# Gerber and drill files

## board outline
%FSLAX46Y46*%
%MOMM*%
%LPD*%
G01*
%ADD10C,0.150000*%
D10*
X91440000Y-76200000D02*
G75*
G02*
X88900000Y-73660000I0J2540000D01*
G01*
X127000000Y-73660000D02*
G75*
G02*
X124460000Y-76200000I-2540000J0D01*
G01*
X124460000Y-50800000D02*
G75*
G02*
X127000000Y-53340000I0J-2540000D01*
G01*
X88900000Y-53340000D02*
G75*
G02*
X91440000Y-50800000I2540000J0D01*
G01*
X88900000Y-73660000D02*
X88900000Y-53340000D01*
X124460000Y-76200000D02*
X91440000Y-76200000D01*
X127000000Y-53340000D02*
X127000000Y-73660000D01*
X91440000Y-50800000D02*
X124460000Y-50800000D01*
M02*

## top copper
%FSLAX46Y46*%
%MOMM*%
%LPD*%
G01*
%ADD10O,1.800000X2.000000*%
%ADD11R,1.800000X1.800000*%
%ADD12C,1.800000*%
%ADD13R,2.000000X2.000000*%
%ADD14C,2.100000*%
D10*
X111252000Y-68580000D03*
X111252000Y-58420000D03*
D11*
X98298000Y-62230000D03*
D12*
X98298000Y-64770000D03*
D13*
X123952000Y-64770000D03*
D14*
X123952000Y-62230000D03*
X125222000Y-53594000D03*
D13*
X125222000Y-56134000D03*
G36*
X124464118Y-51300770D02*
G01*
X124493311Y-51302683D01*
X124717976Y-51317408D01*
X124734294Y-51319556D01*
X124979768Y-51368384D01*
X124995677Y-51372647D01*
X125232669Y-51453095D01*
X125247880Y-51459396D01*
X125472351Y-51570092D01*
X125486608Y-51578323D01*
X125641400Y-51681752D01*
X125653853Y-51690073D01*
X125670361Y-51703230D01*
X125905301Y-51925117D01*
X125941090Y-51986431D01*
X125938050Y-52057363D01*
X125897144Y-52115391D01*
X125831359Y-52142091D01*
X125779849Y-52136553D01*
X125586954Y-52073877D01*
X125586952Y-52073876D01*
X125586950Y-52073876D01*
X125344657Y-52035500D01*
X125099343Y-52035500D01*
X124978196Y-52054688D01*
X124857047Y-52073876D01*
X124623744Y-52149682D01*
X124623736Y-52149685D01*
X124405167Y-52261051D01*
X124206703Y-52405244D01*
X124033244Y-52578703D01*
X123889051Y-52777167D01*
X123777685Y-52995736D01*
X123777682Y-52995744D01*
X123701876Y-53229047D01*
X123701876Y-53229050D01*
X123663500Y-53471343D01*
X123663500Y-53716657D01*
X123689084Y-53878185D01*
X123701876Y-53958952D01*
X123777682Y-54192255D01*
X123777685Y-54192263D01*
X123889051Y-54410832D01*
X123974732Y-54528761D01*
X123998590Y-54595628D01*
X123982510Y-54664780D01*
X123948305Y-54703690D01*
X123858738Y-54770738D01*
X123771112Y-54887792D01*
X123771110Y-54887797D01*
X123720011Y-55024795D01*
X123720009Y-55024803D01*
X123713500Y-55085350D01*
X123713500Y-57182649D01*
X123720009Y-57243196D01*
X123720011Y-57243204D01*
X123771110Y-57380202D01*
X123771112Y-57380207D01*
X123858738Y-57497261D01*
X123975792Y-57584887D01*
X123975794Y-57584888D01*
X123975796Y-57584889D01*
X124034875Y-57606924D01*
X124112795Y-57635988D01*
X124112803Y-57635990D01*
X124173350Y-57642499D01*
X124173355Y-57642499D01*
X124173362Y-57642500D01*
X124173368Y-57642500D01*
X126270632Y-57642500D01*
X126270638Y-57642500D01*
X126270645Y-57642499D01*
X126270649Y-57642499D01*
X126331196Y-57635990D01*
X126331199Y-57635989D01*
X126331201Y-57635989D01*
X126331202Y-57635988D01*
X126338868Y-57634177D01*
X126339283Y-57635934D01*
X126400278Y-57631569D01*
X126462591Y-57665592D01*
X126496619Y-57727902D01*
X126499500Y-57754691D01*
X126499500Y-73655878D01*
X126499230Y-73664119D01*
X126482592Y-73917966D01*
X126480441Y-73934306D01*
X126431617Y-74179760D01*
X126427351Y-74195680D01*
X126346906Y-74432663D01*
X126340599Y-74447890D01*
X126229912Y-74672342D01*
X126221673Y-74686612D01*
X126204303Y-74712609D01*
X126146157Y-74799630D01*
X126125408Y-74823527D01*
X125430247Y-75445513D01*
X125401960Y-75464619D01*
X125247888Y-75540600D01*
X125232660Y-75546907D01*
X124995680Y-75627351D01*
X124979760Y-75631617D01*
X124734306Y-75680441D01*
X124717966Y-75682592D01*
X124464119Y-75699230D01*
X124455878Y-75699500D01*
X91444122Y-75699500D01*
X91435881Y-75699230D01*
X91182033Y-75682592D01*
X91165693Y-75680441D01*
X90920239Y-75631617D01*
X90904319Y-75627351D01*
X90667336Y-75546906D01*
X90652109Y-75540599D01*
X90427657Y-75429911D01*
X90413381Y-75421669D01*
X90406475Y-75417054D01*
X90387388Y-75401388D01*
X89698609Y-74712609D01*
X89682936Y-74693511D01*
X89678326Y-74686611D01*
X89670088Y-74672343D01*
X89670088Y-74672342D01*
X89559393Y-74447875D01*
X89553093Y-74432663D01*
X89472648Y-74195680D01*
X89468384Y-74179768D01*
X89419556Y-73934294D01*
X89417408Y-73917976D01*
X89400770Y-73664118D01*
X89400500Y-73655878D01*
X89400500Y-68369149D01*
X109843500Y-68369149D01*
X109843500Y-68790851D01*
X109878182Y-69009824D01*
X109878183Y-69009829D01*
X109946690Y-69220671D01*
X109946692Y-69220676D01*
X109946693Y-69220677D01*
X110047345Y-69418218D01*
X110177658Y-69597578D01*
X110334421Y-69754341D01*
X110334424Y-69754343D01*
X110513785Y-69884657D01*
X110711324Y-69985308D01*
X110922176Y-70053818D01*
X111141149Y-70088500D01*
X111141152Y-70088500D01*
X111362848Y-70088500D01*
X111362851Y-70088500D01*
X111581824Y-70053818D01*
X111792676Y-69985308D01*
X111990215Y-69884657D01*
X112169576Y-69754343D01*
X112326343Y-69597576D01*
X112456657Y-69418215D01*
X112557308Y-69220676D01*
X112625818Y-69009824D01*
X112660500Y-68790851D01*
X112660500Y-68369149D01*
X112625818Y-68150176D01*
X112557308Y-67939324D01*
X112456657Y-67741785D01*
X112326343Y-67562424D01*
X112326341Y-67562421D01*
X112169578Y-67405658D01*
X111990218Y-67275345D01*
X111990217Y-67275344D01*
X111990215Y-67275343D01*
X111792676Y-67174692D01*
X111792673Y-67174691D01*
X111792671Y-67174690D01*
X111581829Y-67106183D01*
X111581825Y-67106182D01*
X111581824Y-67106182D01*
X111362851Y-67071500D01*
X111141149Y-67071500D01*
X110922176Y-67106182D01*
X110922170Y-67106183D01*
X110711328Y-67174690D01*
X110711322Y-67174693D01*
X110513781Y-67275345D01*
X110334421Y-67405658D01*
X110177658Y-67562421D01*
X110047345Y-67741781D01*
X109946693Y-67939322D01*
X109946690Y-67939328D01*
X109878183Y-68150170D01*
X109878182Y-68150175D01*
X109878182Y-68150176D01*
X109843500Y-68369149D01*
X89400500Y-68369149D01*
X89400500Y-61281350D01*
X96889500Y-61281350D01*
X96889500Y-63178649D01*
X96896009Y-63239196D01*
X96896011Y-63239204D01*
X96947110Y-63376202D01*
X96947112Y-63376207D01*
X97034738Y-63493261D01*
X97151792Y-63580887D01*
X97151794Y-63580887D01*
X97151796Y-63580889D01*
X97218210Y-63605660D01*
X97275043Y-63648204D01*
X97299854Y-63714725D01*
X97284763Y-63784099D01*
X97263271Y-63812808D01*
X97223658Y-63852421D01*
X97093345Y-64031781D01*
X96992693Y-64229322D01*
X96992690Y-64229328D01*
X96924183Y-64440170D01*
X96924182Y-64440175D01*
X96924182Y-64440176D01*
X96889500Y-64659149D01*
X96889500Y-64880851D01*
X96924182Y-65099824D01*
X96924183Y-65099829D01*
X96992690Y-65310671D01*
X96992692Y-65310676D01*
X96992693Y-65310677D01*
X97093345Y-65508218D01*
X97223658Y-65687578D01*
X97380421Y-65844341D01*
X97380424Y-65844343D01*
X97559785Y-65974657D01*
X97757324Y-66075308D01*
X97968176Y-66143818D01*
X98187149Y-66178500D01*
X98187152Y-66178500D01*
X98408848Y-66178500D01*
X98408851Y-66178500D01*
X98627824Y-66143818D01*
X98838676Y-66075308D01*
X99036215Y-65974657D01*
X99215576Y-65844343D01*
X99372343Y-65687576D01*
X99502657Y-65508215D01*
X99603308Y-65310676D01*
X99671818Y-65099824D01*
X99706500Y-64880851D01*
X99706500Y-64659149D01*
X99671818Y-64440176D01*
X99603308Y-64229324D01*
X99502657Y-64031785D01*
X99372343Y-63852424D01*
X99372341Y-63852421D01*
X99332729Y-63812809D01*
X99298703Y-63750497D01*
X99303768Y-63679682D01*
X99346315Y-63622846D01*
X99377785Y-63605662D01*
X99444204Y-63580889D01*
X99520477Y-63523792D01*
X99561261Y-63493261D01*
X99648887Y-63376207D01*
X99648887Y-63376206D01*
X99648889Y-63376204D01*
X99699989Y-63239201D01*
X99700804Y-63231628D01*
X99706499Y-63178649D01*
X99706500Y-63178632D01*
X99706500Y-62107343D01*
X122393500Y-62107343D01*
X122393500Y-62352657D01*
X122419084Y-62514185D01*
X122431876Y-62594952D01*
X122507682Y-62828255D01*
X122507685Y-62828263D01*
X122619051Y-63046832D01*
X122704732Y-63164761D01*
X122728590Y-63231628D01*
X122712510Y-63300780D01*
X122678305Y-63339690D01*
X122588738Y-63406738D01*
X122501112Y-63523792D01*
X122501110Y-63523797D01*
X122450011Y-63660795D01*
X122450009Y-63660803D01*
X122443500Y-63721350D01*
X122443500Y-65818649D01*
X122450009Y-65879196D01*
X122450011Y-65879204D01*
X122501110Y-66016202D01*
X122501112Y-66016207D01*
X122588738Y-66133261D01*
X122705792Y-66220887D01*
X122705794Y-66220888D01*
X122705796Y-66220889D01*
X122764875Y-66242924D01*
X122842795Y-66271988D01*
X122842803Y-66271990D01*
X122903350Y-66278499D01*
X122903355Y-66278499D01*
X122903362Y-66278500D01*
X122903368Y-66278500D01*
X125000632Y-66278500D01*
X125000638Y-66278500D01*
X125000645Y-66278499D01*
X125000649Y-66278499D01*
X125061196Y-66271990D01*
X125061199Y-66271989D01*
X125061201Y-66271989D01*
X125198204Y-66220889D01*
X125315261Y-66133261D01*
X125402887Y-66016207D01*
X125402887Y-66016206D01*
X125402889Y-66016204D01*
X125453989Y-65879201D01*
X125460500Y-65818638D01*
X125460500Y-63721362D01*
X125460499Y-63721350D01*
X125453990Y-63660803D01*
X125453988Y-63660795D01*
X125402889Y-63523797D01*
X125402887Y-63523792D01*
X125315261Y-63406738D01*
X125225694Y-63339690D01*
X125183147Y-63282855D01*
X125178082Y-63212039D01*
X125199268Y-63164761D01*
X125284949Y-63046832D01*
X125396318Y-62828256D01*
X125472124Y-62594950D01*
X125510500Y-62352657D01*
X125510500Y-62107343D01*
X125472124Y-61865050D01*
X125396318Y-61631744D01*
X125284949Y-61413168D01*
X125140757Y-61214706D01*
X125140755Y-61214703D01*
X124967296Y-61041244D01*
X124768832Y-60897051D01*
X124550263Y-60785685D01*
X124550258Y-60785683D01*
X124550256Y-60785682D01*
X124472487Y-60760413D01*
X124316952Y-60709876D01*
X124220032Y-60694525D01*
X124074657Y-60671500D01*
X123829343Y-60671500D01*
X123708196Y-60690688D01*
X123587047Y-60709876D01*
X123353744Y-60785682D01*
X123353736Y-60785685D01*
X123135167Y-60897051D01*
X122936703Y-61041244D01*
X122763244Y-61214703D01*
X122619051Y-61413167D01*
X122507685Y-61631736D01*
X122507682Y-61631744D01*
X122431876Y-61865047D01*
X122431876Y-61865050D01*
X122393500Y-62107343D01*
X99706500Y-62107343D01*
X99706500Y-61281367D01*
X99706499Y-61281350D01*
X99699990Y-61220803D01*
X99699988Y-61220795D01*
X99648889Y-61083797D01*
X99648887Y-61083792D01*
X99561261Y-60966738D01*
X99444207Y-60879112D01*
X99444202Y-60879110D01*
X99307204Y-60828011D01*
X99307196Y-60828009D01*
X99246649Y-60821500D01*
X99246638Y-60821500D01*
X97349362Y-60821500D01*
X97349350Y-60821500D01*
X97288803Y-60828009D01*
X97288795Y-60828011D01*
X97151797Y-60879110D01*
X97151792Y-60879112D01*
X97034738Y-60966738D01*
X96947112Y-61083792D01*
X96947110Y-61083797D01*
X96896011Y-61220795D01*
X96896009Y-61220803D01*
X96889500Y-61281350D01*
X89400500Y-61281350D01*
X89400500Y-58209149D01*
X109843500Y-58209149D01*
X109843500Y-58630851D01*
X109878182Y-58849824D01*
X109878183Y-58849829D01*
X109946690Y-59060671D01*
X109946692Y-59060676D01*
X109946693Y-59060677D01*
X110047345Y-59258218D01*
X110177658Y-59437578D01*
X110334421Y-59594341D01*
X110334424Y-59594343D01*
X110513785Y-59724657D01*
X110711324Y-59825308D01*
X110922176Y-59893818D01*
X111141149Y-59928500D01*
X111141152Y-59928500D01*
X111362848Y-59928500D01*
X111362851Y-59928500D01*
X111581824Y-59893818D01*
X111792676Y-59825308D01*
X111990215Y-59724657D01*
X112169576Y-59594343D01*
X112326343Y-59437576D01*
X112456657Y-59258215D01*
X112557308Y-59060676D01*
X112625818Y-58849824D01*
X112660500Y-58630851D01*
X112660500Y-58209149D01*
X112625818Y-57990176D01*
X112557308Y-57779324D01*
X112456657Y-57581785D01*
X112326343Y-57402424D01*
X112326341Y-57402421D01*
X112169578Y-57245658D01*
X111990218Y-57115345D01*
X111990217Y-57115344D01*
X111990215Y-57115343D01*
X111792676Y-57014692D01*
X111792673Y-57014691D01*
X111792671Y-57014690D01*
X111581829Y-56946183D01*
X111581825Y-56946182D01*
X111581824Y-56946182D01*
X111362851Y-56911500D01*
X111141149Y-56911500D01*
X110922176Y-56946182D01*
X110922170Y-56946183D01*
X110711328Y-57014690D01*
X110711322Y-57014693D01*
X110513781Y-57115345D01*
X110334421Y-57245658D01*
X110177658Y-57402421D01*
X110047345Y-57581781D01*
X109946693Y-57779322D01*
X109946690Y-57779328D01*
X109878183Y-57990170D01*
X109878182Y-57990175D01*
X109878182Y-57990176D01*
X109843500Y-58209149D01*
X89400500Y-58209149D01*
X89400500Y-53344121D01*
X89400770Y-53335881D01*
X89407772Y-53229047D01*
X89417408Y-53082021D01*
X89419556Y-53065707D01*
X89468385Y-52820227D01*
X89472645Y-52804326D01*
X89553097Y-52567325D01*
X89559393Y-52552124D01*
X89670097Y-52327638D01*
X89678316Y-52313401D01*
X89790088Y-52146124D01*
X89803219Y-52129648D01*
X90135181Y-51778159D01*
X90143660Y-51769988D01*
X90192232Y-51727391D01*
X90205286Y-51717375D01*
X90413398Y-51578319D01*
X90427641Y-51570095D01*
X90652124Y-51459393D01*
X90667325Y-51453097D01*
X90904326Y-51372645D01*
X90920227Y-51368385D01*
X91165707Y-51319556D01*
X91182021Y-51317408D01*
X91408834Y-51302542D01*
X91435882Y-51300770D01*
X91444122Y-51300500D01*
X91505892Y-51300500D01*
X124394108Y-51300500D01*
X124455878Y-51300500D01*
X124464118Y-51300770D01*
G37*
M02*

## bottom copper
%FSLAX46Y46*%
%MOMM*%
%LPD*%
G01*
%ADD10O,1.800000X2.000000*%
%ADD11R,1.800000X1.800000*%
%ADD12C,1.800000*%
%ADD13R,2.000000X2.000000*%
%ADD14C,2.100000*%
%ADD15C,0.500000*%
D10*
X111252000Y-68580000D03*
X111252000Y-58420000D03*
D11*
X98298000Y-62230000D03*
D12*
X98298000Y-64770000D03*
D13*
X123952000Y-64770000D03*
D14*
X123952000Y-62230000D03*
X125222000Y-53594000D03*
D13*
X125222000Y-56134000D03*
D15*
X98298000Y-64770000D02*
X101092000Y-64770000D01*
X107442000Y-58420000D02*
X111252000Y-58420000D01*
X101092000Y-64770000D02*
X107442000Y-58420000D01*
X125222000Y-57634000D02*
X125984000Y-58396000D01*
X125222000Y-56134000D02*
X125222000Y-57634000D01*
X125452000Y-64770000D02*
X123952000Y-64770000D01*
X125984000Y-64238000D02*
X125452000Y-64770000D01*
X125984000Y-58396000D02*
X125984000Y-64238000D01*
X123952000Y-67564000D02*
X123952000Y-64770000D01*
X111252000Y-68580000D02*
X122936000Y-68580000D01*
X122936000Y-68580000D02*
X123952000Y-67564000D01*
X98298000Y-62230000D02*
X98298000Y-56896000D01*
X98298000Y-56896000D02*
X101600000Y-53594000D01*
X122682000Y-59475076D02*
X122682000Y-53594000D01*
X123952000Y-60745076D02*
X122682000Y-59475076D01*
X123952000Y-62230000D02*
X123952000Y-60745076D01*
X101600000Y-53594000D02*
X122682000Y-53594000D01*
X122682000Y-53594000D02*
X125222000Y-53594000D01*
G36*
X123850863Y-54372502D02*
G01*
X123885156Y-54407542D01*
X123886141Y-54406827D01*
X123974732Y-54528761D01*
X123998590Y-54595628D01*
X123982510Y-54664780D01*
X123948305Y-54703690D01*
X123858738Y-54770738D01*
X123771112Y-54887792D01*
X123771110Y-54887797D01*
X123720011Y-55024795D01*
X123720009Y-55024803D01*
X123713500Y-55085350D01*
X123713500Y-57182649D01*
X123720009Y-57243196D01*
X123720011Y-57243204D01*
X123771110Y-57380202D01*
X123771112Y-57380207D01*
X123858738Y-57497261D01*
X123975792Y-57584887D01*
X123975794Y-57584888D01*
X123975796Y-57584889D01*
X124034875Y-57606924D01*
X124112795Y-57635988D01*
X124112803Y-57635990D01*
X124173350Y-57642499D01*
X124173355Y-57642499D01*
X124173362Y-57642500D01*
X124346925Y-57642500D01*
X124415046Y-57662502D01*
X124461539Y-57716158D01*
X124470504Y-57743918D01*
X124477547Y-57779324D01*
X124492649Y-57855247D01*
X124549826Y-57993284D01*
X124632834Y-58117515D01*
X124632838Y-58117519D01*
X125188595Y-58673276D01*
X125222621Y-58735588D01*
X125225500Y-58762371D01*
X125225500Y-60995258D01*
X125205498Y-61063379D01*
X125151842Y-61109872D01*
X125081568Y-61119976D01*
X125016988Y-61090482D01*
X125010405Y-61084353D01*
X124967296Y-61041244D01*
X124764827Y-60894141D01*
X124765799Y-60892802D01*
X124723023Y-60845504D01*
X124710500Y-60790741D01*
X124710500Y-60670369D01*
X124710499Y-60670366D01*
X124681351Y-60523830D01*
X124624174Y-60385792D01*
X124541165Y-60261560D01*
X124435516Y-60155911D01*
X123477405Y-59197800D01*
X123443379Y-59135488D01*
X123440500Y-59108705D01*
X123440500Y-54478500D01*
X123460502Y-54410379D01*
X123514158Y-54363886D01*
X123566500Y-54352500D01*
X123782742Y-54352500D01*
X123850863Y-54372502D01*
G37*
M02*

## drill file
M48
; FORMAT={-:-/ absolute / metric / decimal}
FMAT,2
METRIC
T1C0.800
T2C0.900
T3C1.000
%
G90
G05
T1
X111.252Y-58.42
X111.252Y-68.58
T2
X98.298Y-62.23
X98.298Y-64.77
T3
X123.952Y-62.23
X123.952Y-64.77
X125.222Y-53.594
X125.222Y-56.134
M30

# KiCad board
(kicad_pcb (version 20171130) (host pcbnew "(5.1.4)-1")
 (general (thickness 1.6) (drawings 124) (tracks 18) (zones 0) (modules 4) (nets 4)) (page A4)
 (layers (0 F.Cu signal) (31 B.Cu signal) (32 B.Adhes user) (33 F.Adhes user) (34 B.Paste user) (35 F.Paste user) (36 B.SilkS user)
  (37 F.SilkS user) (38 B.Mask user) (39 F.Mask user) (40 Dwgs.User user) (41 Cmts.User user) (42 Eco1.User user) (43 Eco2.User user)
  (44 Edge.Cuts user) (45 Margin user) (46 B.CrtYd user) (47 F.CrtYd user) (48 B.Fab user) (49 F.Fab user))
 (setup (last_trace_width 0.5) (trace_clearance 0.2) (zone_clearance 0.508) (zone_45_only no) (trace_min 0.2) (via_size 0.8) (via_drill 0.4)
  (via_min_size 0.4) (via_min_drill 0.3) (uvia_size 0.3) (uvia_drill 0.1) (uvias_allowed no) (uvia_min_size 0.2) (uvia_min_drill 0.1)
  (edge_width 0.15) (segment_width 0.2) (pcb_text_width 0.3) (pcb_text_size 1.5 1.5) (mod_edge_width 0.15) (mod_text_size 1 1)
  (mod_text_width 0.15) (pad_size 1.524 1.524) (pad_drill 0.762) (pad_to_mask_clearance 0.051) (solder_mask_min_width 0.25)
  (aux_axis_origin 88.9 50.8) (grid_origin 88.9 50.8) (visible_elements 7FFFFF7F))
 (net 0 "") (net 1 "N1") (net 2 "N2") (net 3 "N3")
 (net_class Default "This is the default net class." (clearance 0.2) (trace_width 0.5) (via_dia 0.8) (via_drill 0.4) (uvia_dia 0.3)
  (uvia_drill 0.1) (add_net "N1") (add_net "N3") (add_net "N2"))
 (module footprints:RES (layer F.Cu) (at 111.252 68.58 90)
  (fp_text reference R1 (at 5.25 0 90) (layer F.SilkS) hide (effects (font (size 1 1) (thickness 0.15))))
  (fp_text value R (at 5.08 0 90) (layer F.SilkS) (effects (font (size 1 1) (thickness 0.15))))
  (pad 1 thru_hole oval (at 0 0 90) (size 2 1.8) (drill 0.8) (layers *.Cu *.Mask) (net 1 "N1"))
  (pad 2 thru_hole oval (at 10.16 0 90) (size 2 1.8) (drill 0.8) (layers *.Cu *.Mask) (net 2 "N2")))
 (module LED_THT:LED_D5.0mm (layer F.Cu) (at 98.298 62.23 270)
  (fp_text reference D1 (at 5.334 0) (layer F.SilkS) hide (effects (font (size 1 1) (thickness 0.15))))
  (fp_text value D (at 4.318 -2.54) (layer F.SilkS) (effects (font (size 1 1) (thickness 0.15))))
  (pad 1 thru_hole rect (at 0 0 270) (size 1.8 1.8) (drill 0.9) (layers *.Cu *.Mask) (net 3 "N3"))
  (pad 2 thru_hole circle (at 2.54 0 270) (size 1.8 1.8) (drill 0.9) (layers *.Cu *.Mask) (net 2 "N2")))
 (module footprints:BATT (layer F.Cu) (at 123.952 63.5)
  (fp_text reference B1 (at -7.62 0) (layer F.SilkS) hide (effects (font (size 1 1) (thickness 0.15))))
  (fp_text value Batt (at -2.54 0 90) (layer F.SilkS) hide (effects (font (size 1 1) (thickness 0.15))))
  (pad 1 thru_hole rect (at 0 1.27) (size 2 2) (drill 1) (layers *.Cu *.Mask) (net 1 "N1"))
  (pad 2 thru_hole circle (at 0 -1.27) (size 2.1 2.1) (drill 1) (layers *.Cu *.Mask) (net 3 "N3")))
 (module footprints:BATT (layer B.Cu) (at 125.222 54.864 180)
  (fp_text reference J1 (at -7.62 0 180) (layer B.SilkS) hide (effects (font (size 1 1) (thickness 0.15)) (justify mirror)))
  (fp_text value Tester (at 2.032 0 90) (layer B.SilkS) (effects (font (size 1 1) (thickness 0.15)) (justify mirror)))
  (pad 2 thru_hole circle (at 0 1.27 180) (size 2.1 2.1) (drill 1) (layers *.Cu *.Mask) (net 3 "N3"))
  (pad 1 thru_hole rect (at 0 -1.27 180) (size 2 2) (drill 1) (layers *.Cu *.Mask) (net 1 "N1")))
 (gr_arc (start 91.44 73.66) (end 88.9 73.66) (angle -90) (layer Edge.Cuts) (width 0.15))
 (gr_arc (start 124.46 73.66) (end 124.46 76.2) (angle -90) (layer Edge.Cuts) (width 0.15))
 (gr_arc (start 124.46 53.34) (end 127 53.34) (angle -90) (layer Edge.Cuts) (width 0.15))
 (gr_arc (start 91.44 53.34) (end 91.44 50.8) (angle -90) (layer Edge.Cuts) (width 0.15))
 (gr_line (start 88.9 73.66) (end 88.9 53.34) (layer Edge.Cuts) (width 0.15))
 (gr_line (start 124.46 76.2) (end 91.44 76.2) (layer Edge.Cuts) (width 0.15))
 (gr_line (start 127 53.34) (end 127 73.66) (layer Edge.Cuts) (width 0.15))
 (gr_line (start 91.44 50.8) (end 124.46 50.8) (layer Edge.Cuts) (width 0.15))
 (segment (start 98.298 64.77) (end 101.092 64.77) (width 0.5) (layer B.Cu) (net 2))
 (segment (start 107.442 58.42) (end 111.252 58.42) (width 0.5) (layer B.Cu) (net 2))
 (segment (start 101.092 64.77) (end 107.442 58.42) (width 0.5) (layer B.Cu) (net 2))
 (segment (start 125.222 57.634) (end 125.984 58.396) (width 0.5) (layer B.Cu) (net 1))
 (segment (start 125.222 56.134) (end 125.222 57.634) (width 0.5) (layer B.Cu) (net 1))
 (segment (start 125.452 64.77) (end 123.952 64.77) (width 0.5) (layer B.Cu) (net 1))
 (segment (start 125.984 64.238) (end 125.452 64.77) (width 0.5) (layer B.Cu) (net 1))
 (segment (start 125.984 58.396) (end 125.984 64.238) (width 0.5) (layer B.Cu) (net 1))
 (segment (start 123.952 67.564) (end 123.952 64.77) (width 0.5) (layer B.Cu) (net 1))
 (segment (start 111.252 68.58) (end 122.936 68.58) (width 0.5) (layer B.Cu) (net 1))
 (segment (start 122.936 68.58) (end 123.952 67.564) (width 0.5) (layer B.Cu) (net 1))
 (segment (start 98.298 62.23) (end 98.298 56.896) (width 0.5) (layer B.Cu) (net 3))
 (segment (start 98.298 56.896) (end 101.6 53.594) (width 0.5) (layer B.Cu) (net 3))
 (segment (start 122.682 59.475076) (end 122.682 53.594) (width 0.5) (layer B.Cu) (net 3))
 (segment (start 123.952 60.745076) (end 122.682 59.475076) (width 0.5) (layer B.Cu) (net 3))
 (segment (start 123.952 62.23) (end 123.952 60.745076) (width 0.5) (layer B.Cu) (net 3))
 (segment (start 101.6 53.594) (end 122.682 53.594) (width 0.5) (layer B.Cu) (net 3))
 (segment (start 122.682 53.594) (end 125.222 53.594) (width 0.5) (layer B.Cu) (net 3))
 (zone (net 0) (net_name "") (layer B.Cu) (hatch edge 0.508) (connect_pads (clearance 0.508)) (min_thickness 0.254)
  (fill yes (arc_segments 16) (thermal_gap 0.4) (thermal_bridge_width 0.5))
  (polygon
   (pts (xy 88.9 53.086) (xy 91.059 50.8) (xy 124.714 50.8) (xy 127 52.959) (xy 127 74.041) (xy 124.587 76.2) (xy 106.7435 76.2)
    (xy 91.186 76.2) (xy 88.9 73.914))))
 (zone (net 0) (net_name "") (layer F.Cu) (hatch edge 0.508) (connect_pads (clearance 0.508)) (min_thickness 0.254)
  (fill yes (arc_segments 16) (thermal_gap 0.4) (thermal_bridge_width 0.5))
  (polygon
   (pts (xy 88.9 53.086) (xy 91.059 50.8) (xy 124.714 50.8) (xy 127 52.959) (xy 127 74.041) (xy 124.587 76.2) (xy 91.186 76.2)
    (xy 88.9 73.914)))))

